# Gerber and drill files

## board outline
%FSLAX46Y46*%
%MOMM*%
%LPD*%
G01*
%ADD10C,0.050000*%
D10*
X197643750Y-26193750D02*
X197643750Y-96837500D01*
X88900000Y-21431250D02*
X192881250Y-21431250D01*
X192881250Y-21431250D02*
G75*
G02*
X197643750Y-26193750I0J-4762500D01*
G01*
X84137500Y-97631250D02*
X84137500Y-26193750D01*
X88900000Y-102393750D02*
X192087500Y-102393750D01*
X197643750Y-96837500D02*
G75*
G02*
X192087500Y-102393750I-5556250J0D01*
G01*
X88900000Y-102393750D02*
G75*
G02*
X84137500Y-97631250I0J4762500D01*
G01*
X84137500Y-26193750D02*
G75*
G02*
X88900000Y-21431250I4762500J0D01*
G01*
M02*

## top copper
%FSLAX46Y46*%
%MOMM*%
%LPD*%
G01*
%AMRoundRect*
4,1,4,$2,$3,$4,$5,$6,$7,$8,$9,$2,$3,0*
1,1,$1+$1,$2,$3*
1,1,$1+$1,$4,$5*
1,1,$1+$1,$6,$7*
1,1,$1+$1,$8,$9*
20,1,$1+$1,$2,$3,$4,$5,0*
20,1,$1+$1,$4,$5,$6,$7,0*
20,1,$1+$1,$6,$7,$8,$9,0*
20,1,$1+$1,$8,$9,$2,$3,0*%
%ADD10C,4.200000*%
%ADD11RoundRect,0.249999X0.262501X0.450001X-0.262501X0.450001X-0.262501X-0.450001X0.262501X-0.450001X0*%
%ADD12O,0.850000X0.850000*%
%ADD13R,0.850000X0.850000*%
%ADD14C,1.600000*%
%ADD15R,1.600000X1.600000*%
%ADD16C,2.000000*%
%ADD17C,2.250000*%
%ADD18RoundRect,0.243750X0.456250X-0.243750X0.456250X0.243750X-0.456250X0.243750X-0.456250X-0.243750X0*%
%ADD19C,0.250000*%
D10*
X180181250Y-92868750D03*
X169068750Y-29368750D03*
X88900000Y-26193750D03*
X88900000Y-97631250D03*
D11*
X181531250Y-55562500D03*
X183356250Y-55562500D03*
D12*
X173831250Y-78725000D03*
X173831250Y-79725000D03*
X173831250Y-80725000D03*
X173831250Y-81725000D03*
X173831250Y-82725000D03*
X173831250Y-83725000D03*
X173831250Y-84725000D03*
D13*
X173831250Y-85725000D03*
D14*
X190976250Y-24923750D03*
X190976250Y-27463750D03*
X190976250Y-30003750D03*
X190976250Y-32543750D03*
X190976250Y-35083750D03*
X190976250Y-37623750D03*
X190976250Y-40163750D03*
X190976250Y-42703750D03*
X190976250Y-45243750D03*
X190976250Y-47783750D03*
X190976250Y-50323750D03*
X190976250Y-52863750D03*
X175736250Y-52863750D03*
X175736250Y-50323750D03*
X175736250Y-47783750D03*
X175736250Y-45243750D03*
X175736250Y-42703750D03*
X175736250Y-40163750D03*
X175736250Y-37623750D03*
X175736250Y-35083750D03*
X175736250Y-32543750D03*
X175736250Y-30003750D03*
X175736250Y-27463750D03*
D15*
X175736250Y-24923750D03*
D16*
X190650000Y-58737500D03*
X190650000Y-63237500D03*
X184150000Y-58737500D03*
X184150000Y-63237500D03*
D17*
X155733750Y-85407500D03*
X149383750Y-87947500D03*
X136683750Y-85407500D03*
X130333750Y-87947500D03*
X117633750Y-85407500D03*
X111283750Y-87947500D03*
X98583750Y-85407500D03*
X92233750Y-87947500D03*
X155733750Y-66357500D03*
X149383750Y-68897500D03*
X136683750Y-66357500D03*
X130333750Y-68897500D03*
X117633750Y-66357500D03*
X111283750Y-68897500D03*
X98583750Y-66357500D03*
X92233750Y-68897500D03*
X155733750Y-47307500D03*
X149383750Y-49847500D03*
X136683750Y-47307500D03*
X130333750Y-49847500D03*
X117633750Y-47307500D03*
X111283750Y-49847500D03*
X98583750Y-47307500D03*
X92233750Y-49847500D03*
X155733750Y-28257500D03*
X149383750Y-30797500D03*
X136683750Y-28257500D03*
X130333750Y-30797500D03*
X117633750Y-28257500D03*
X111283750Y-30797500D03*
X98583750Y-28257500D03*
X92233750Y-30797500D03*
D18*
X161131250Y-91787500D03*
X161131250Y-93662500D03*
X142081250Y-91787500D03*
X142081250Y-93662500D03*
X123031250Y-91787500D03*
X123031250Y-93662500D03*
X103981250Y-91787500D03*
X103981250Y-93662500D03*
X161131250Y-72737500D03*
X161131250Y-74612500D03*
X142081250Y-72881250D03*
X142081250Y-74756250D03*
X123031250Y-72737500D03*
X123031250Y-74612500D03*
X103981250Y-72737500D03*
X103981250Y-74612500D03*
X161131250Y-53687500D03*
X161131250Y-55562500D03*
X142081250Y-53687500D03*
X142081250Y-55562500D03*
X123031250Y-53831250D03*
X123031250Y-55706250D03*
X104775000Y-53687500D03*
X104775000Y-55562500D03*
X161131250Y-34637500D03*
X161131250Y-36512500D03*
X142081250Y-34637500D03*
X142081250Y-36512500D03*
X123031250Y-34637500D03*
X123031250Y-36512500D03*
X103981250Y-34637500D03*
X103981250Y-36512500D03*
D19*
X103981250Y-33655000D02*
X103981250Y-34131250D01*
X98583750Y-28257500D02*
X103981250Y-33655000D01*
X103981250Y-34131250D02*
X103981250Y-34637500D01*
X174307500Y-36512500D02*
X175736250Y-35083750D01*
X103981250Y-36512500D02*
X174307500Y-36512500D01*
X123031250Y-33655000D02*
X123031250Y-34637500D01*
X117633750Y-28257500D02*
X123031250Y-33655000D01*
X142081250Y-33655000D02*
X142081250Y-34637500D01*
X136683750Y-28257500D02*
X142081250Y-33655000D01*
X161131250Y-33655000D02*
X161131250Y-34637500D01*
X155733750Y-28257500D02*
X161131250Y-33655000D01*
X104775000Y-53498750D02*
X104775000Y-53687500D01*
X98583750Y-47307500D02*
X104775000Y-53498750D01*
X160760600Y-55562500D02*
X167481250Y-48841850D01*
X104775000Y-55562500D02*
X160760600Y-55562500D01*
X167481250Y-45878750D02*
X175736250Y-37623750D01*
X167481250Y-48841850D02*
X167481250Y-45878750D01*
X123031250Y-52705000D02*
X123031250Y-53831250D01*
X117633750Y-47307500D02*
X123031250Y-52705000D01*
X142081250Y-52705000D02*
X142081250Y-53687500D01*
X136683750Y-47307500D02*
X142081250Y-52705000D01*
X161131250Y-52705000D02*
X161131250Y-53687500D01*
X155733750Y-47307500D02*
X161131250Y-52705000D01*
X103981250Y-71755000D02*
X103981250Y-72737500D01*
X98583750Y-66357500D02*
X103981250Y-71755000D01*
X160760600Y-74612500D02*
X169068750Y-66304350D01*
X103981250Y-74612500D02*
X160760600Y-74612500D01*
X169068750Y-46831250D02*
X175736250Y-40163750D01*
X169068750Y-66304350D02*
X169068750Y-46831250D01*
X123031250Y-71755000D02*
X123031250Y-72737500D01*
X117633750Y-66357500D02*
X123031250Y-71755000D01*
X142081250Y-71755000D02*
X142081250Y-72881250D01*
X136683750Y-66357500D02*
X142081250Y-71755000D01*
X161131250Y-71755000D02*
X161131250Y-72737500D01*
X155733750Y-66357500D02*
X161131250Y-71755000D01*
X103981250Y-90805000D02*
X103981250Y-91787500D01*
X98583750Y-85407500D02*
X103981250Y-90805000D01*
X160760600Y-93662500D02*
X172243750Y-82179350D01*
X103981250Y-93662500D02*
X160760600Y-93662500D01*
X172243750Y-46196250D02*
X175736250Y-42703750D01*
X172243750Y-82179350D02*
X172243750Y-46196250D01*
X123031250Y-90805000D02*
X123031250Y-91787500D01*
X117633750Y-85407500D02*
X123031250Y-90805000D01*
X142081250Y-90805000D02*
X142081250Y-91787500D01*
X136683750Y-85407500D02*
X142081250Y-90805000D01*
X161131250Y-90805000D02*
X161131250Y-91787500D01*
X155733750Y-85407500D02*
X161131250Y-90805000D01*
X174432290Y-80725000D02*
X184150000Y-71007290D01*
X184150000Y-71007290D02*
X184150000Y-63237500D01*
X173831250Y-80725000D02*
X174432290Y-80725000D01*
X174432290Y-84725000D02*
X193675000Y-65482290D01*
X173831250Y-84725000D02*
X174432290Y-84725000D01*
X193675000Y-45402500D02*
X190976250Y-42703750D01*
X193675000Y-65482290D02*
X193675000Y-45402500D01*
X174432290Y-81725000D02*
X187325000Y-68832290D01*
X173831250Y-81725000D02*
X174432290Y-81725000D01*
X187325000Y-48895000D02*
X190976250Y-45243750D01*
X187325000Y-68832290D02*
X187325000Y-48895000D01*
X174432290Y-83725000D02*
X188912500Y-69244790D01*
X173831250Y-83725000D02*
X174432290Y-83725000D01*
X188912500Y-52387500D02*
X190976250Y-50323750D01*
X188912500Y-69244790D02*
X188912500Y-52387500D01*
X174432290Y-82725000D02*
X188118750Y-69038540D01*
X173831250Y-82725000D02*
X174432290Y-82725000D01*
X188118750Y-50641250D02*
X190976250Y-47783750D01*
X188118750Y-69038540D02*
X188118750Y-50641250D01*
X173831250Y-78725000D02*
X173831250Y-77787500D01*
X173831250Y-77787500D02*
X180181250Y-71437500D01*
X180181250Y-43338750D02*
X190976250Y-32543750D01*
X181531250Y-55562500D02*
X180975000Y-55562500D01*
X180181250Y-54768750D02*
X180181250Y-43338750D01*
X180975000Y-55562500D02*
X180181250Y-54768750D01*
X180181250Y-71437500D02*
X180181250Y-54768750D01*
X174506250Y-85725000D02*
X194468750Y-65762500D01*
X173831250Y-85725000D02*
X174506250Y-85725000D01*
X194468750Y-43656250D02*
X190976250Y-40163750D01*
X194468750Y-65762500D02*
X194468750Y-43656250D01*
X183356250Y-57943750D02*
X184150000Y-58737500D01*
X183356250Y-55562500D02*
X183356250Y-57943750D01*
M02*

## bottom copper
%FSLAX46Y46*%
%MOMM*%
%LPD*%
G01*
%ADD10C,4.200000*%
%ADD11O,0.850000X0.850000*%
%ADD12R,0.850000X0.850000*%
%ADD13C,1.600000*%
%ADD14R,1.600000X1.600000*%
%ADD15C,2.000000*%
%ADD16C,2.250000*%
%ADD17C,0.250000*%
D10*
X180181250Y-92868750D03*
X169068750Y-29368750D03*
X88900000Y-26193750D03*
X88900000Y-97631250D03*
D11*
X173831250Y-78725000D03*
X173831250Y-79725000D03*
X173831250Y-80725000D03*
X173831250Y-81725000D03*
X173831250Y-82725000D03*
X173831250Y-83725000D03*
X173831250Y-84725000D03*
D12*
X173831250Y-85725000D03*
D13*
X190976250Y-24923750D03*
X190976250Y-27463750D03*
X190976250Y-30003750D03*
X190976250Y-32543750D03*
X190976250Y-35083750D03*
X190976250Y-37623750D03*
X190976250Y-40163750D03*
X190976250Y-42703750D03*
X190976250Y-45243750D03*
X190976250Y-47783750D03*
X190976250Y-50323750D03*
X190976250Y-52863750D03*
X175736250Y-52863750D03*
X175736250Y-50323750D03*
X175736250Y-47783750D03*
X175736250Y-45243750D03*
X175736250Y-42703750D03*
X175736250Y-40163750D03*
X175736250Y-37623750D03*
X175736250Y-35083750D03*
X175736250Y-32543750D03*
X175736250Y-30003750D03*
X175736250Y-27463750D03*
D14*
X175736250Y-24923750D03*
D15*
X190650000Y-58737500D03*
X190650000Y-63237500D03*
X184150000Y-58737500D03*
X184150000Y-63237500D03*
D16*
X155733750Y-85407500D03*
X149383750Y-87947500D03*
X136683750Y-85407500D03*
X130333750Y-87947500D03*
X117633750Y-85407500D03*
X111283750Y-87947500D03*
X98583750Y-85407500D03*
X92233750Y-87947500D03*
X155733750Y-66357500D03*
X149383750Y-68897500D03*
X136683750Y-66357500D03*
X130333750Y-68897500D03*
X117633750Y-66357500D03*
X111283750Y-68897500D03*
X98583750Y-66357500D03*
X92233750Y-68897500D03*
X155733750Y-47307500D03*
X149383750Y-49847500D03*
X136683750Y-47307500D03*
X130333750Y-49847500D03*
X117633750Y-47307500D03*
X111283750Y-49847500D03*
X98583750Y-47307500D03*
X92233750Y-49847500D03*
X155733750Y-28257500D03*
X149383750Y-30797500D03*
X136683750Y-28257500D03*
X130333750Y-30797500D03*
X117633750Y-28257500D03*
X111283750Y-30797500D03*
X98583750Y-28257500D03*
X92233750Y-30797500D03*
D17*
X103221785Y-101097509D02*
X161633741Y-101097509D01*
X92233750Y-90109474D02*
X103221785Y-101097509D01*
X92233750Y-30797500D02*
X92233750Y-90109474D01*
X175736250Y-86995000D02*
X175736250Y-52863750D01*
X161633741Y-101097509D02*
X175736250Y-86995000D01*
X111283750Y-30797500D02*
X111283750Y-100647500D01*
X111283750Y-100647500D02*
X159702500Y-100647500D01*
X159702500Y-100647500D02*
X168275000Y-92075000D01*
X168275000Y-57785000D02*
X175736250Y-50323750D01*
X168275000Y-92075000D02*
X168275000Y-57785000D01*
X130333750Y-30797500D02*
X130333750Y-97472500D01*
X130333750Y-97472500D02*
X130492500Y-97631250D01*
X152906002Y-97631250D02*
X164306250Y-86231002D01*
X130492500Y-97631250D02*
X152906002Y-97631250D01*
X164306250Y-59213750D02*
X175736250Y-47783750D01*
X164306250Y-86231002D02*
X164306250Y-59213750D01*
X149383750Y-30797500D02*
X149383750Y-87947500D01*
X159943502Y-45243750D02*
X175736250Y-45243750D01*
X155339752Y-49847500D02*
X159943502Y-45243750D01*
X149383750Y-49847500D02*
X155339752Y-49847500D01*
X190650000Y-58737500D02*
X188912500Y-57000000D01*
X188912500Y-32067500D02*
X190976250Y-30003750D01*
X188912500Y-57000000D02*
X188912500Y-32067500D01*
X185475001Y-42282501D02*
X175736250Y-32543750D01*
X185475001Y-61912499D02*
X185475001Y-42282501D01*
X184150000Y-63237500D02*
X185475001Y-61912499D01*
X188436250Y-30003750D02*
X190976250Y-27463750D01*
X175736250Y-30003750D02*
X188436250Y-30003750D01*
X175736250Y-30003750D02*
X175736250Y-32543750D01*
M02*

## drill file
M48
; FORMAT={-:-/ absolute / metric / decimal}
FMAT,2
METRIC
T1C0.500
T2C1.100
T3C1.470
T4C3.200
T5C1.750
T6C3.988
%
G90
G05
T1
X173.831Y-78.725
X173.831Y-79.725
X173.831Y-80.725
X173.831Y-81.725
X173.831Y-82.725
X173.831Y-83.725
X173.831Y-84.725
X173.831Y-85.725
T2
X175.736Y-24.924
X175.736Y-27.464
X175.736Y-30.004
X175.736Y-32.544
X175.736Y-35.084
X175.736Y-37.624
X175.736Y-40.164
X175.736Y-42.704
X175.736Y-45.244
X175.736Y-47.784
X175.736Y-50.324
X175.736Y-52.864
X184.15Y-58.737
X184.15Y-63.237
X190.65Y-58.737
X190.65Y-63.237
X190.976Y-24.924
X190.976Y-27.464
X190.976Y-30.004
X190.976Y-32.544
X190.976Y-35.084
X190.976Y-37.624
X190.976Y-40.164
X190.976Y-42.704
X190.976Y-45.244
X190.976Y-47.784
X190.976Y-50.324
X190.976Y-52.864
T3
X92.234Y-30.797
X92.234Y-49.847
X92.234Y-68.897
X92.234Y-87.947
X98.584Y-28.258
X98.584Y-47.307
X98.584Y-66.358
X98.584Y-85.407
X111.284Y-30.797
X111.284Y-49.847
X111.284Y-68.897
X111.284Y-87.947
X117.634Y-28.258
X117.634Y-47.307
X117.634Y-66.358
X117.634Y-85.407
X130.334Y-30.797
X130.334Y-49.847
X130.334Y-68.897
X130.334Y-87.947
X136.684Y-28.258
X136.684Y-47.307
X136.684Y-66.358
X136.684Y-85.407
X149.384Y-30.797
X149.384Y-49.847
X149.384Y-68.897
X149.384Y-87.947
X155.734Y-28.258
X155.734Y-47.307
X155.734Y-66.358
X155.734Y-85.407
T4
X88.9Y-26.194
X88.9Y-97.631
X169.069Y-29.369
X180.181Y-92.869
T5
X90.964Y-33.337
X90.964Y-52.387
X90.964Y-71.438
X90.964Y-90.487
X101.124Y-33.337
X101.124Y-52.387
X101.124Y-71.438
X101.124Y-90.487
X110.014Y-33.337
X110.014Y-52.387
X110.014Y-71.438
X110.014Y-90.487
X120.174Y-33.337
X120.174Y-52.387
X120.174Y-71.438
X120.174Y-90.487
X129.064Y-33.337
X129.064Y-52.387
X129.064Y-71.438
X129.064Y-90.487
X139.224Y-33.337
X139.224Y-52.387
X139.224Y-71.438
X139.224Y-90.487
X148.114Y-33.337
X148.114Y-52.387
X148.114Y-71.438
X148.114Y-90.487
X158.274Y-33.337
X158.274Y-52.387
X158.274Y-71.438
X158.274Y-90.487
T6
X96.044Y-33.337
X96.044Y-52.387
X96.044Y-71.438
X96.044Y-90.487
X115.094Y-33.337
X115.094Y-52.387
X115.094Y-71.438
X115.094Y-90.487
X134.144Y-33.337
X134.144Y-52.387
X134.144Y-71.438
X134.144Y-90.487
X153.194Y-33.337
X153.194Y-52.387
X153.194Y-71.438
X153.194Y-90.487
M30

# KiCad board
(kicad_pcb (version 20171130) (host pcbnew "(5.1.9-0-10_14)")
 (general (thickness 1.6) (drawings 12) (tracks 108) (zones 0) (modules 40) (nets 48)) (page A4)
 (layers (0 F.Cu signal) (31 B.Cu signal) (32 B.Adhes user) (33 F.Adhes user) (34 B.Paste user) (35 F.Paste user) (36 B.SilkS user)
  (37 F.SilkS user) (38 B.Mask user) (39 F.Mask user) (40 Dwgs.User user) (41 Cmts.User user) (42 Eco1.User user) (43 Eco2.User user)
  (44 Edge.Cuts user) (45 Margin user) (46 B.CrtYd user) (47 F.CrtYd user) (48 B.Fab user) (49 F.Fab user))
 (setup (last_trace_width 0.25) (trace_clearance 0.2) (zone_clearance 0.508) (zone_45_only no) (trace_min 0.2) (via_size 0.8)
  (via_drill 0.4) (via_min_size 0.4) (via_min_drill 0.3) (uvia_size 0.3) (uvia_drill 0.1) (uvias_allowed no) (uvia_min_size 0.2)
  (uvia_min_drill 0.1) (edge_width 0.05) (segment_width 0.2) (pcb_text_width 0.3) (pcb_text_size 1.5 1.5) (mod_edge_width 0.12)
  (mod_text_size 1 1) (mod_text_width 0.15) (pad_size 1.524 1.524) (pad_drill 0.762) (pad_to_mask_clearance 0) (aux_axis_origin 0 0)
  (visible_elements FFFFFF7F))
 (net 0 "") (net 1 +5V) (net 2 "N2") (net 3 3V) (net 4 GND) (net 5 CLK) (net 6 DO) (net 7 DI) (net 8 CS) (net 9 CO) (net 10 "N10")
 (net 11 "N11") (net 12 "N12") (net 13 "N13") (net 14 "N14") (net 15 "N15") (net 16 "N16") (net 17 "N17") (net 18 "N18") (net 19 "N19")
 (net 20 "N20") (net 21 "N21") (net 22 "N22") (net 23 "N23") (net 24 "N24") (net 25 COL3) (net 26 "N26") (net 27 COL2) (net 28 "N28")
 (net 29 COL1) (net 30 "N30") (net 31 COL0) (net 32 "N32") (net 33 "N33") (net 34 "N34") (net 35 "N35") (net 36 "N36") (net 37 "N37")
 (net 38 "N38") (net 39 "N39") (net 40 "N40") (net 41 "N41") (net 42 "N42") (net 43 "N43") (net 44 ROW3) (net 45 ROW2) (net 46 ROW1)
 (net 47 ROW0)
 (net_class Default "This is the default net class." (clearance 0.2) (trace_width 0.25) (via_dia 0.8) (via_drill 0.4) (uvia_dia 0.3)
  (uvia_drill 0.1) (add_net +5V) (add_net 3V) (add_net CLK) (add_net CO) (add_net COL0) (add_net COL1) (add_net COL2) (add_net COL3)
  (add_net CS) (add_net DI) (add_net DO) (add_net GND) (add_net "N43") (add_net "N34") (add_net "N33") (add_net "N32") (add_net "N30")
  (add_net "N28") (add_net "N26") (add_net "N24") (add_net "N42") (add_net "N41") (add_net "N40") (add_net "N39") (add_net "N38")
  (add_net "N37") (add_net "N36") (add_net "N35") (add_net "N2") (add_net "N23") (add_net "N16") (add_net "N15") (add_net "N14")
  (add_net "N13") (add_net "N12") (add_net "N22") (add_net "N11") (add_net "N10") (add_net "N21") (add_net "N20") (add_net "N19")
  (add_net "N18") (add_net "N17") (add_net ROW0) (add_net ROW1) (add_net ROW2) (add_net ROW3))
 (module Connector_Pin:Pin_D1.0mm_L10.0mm (layer F.Cu) (at 180.18125 92.86875)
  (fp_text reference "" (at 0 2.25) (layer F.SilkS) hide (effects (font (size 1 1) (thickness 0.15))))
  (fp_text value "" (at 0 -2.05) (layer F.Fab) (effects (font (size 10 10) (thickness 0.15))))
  (pad "" thru_hole circle (at 0 0) (size 4.2 4.2) (drill 3.2) (layers *.Cu *.Mask)))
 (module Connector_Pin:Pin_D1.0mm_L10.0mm (layer F.Cu) (at 169.06875 29.36875)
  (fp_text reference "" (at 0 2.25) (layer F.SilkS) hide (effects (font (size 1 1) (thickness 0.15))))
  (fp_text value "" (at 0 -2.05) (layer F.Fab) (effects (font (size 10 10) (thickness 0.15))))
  (pad "" thru_hole circle (at 0 0) (size 4.2 4.2) (drill 3.2) (layers *.Cu *.Mask)))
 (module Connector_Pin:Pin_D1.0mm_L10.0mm (layer F.Cu) (at 88.9 26.19375)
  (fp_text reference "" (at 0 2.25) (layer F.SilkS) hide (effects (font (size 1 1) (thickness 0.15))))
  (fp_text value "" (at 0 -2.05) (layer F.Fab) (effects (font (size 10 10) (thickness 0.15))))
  (pad "" thru_hole circle (at 0 0) (size 4.2 4.2) (drill 3.2) (layers *.Cu *.Mask)))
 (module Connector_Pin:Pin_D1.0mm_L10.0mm (layer F.Cu) (at 88.9 97.63125)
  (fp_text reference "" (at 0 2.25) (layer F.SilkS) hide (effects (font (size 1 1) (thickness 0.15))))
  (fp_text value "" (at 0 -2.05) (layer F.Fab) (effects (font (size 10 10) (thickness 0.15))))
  (pad "" thru_hole circle (at 0 0) (size 4.2 4.2) (drill 3.2) (layers *.Cu *.Mask)))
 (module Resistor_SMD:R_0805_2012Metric (layer F.Cu) (at 182.44375 55.5625 180)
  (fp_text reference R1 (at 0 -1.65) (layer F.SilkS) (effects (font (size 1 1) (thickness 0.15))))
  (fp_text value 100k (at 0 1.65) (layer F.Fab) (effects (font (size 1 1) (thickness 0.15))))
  (pad 2 smd roundrect (at 0.9125 0 180) (size 1.025 1.4) (layers F.Cu F.Paste F.Mask) (roundrect_rratio 0.2439014634146341) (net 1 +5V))
  (pad 1 smd roundrect (at -0.9125 0 180) (size 1.025 1.4) (layers F.Cu F.Paste F.Mask) (roundrect_rratio 0.2439014634146341) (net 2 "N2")))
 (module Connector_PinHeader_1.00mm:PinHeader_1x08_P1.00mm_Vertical (layer F.Cu) (at 173.83125 85.725 180)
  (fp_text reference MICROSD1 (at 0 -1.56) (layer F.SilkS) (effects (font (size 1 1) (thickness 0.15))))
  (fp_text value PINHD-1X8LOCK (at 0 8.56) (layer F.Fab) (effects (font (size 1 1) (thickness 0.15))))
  (pad 8 thru_hole oval (at 0 7 180) (size 0.85 0.85) (drill 0.5) (layers *.Cu *.Mask) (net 1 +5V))
  (pad 7 thru_hole oval (at 0 6 180) (size 0.85 0.85) (drill 0.5) (layers *.Cu *.Mask) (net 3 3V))
  (pad 6 thru_hole oval (at 0 5 180) (size 0.85 0.85) (drill 0.5) (layers *.Cu *.Mask) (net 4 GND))
  (pad 5 thru_hole oval (at 0 4 180) (size 0.85 0.85) (drill 0.5) (layers *.Cu *.Mask) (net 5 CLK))
  (pad 4 thru_hole oval (at 0 3 180) (size 0.85 0.85) (drill 0.5) (layers *.Cu *.Mask) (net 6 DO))
  (pad 3 thru_hole oval (at 0 2 180) (size 0.85 0.85) (drill 0.5) (layers *.Cu *.Mask) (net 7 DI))
  (pad 2 thru_hole oval (at 0 1 180) (size 0.85 0.85) (drill 0.5) (layers *.Cu *.Mask) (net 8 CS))
  (pad 1 thru_hole rect (at 0 0 180) (size 0.85 0.85) (drill 0.5) (layers *.Cu *.Mask) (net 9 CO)))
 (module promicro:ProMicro (layer F.Cu) (at 183.35625 38.89375 270)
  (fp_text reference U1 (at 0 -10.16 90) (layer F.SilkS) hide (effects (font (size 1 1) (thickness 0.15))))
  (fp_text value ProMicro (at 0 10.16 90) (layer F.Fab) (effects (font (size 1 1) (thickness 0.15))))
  (pad 24 thru_hole circle (at -13.97 -7.62 270) (size 1.6 1.6) (drill 1.1) (layers *.Cu *.Mask F.SilkS) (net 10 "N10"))
  (pad 23 thru_hole circle (at -11.43 -7.62 270) (size 1.6 1.6) (drill 1.1) (layers *.Cu *.Mask F.SilkS) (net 4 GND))
  (pad 22 thru_hole circle (at -8.89 -7.62 270) (size 1.6 1.6) (drill 1.1) (layers *.Cu *.Mask F.SilkS) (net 2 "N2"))
  (pad 21 thru_hole circle (at -6.35 -7.62 270) (size 1.6 1.6) (drill 1.1) (layers *.Cu *.Mask F.SilkS) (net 1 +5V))
  (pad 20 thru_hole circle (at -3.81 -7.62 270) (size 1.6 1.6) (drill 1.1) (layers *.Cu *.Mask F.SilkS) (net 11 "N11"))
  (pad 19 thru_hole circle (at -1.27 -7.62 270) (size 1.6 1.6) (drill 1.1) (layers *.Cu *.Mask F.SilkS) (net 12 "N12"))
  (pad 18 thru_hole circle (at 1.27 -7.62 270) (size 1.6 1.6) (drill 1.1) (layers *.Cu *.Mask F.SilkS) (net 9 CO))
  (pad 17 thru_hole circle (at 3.81 -7.62 270) (size 1.6 1.6) (drill 1.1) (layers *.Cu *.Mask F.SilkS) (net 8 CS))
  (pad 16 thru_hole circle (at 6.35 -7.62 270) (size 1.6 1.6) (drill 1.1) (layers *.Cu *.Mask F.SilkS) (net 5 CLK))
  (pad 15 thru_hole circle (at 8.89 -7.62 270) (size 1.6 1.6) (drill 1.1) (layers *.Cu *.Mask F.SilkS) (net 6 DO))
  (pad 14 thru_hole circle (at 11.43 -7.62 270) (size 1.6 1.6) (drill 1.1) (layers *.Cu *.Mask F.SilkS) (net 7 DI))
  (pad 13 thru_hole circle (at 13.97 -7.62 270) (size 1.6 1.6) (drill 1.1) (layers *.Cu *.Mask F.SilkS) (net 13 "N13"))
  (pad 12 thru_hole circle (at 13.97 7.62 270) (size 1.6 1.6) (drill 1.1) (layers *.Cu *.Mask F.SilkS) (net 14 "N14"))
  (pad 11 thru_hole circle (at 11.43 7.62 270) (size 1.6 1.6) (drill 1.1) (layers *.Cu *.Mask F.SilkS) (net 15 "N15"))
  (pad 10 thru_hole circle (at 8.89 7.62 270) (size 1.6 1.6) (drill 1.1) (layers *.Cu *.Mask F.SilkS) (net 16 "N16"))
  (pad 9 thru_hole circle (at 6.35 7.62 270) (size 1.6 1.6) (drill 1.1) (layers *.Cu *.Mask F.SilkS) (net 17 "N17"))
  (pad 8 thru_hole circle (at 3.81 7.62 270) (size 1.6 1.6) (drill 1.1) (layers *.Cu *.Mask F.SilkS) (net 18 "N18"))
  (pad 7 thru_hole circle (at 1.27 7.62 270) (size 1.6 1.6) (drill 1.1) (layers *.Cu *.Mask F.SilkS) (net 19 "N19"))
  (pad 6 thru_hole circle (at -1.27 7.62 270) (size 1.6 1.6) (drill 1.1) (layers *.Cu *.Mask F.SilkS) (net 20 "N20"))
  (pad 5 thru_hole circle (at -3.81 7.62 270) (size 1.6 1.6) (drill 1.1) (layers *.Cu *.Mask F.SilkS) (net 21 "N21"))
  (pad 4 thru_hole circle (at -6.35 7.62 270) (size 1.6 1.6) (drill 1.1) (layers *.Cu *.Mask F.SilkS) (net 4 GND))
  (pad 3 thru_hole circle (at -8.89 7.62 270) (size 1.6 1.6) (drill 1.1) (layers *.Cu *.Mask F.SilkS) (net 4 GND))
  (pad 2 thru_hole circle (at -11.43 7.62 270) (size 1.6 1.6) (drill 1.1) (layers *.Cu *.Mask F.SilkS) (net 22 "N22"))
  (pad 1 thru_hole rect (at -13.97 7.62 270) (size 1.6 1.6) (drill 1.1) (layers *.Cu *.Mask F.SilkS) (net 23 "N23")))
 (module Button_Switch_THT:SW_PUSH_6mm (layer F.Cu) (at 184.15 58.7375)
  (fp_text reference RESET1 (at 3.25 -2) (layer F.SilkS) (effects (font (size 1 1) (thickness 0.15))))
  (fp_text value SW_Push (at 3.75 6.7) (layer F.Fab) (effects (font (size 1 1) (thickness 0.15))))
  (pad 1 thru_hole circle (at 6.5 0 90) (size 2 2) (drill 1.1) (layers *.Cu *.Mask) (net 2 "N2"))
  (pad 2 thru_hole circle (at 6.5 4.5 90) (size 2 2) (drill 1.1) (layers *.Cu *.Mask) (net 4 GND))
  (pad 1 thru_hole circle (at 0 0 90) (size 2 2) (drill 1.1) (layers *.Cu *.Mask) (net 2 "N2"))
  (pad 2 thru_hole circle (at 0 4.5 90) (size 2 2) (drill 1.1) (layers *.Cu *.Mask) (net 4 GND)))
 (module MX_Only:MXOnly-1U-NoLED (layer F.Cu) (at 153.19375 90.4875)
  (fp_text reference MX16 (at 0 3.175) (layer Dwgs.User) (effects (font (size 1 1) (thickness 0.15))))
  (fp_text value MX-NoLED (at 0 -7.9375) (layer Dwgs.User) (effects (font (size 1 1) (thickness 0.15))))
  (pad 2 thru_hole circle (at 2.54 -5.08) (size 2.25 2.25) (drill 1.47) (layers *.Cu B.Mask) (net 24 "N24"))
  (pad "" np_thru_hole circle (at 0 0) (size 3.9878 3.9878) (drill 3.9878) (layers *.Cu *.Mask))
  (pad 1 thru_hole circle (at -3.81 -2.54) (size 2.25 2.25) (drill 1.47) (layers *.Cu B.Mask) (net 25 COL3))
  (pad "" np_thru_hole circle (at -5.08 0 48.0996) (size 1.75 1.75) (drill 1.75) (layers *.Cu *.Mask))
  (pad "" np_thru_hole circle (at 5.08 0 48.0996) (size 1.75 1.75) (drill 1.75) (layers *.Cu *.Mask)))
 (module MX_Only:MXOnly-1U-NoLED (layer F.Cu) (at 134.14375 90.4875)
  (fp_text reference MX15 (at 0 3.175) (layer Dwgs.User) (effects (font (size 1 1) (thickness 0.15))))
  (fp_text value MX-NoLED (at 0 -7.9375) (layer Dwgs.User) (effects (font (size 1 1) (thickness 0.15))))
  (pad 2 thru_hole circle (at 2.54 -5.08) (size 2.25 2.25) (drill 1.47) (layers *.Cu B.Mask) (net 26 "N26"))
  (pad "" np_thru_hole circle (at 0 0) (size 3.9878 3.9878) (drill 3.9878) (layers *.Cu *.Mask))
  (pad 1 thru_hole circle (at -3.81 -2.54) (size 2.25 2.25) (drill 1.47) (layers *.Cu B.Mask) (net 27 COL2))
  (pad "" np_thru_hole circle (at -5.08 0 48.0996) (size 1.75 1.75) (drill 1.75) (layers *.Cu *.Mask))
  (pad "" np_thru_hole circle (at 5.08 0 48.0996) (size 1.75 1.75) (drill 1.75) (layers *.Cu *.Mask)))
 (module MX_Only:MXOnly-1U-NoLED (layer F.Cu) (at 115.09375 90.4875)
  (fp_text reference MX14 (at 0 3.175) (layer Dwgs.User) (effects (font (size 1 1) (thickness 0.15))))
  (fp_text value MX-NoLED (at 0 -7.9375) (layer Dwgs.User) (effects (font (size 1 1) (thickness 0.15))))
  (pad 2 thru_hole circle (at 2.54 -5.08) (size 2.25 2.25) (drill 1.47) (layers *.Cu B.Mask) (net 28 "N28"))
  (pad "" np_thru_hole circle (at 0 0) (size 3.9878 3.9878) (drill 3.9878) (layers *.Cu *.Mask))
  (pad 1 thru_hole circle (at -3.81 -2.54) (size 2.25 2.25) (drill 1.47) (layers *.Cu B.Mask) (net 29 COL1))
  (pad "" np_thru_hole circle (at -5.08 0 48.0996) (size 1.75 1.75) (drill 1.75) (layers *.Cu *.Mask))
  (pad "" np_thru_hole circle (at 5.08 0 48.0996) (size 1.75 1.75) (drill 1.75) (layers *.Cu *.Mask)))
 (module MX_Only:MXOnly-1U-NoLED (layer F.Cu) (at 96.04375 90.4875)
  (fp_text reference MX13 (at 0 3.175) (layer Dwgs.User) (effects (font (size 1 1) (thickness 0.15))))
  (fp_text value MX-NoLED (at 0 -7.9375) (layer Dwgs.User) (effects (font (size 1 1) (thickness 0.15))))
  (pad 2 thru_hole circle (at 2.54 -5.08) (size 2.25 2.25) (drill 1.47) (layers *.Cu B.Mask) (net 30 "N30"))
  (pad "" np_thru_hole circle (at 0 0) (size 3.9878 3.9878) (drill 3.9878) (layers *.Cu *.Mask))
  (pad 1 thru_hole circle (at -3.81 -2.54) (size 2.25 2.25) (drill 1.47) (layers *.Cu B.Mask) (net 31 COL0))
  (pad "" np_thru_hole circle (at -5.08 0 48.0996) (size 1.75 1.75) (drill 1.75) (layers *.Cu *.Mask))
  (pad "" np_thru_hole circle (at 5.08 0 48.0996) (size 1.75 1.75) (drill 1.75) (layers *.Cu *.Mask)))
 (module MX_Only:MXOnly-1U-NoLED (layer F.Cu) (at 153.19375 71.4375)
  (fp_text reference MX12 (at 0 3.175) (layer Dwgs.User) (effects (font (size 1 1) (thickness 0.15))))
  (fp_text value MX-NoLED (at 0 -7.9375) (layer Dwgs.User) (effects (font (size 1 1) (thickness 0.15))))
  (pad 2 thru_hole circle (at 2.54 -5.08) (size 2.25 2.25) (drill 1.47) (layers *.Cu B.Mask) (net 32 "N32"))
  (pad "" np_thru_hole circle (at 0 0) (size 3.9878 3.9878) (drill 3.9878) (layers *.Cu *.Mask))
  (pad 1 thru_hole circle (at -3.81 -2.54) (size 2.25 2.25) (drill 1.47) (layers *.Cu B.Mask) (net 25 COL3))
  (pad "" np_thru_hole circle (at -5.08 0 48.0996) (size 1.75 1.75) (drill 1.75) (layers *.Cu *.Mask))
  (pad "" np_thru_hole circle (at 5.08 0 48.0996) (size 1.75 1.75) (drill 1.75) (layers *.Cu *.Mask)))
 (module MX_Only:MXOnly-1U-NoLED (layer F.Cu) (at 134.14375 71.4375)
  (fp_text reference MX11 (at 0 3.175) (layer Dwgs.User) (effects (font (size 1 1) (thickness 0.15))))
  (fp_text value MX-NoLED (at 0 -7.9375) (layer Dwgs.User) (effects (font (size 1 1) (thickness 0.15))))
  (pad 2 thru_hole circle (at 2.54 -5.08) (size 2.25 2.25) (drill 1.47) (layers *.Cu B.Mask) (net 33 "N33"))
  (pad "" np_thru_hole circle (at 0 0) (size 3.9878 3.9878) (drill 3.9878) (layers *.Cu *.Mask))
  (pad 1 thru_hole circle (at -3.81 -2.54) (size 2.25 2.25) (drill 1.47) (layers *.Cu B.Mask) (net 27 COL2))
  (pad "" np_thru_hole circle (at -5.08 0 48.0996) (size 1.75 1.75) (drill 1.75) (layers *.Cu *.Mask))
  (pad "" np_thru_hole circle (at 5.08 0 48.0996) (size 1.75 1.75) (drill 1.75) (layers *.Cu *.Mask)))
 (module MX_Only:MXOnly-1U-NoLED (layer F.Cu) (at 115.09375 71.4375)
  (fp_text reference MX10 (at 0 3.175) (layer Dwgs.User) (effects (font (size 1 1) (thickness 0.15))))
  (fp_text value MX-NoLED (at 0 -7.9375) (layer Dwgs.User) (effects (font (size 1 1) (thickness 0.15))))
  (pad 2 thru_hole circle (at 2.54 -5.08) (size 2.25 2.25) (drill 1.47) (layers *.Cu B.Mask) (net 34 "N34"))
  (pad "" np_thru_hole circle (at 0 0) (size 3.9878 3.9878) (drill 3.9878) (layers *.Cu *.Mask))
  (pad 1 thru_hole circle (at -3.81 -2.54) (size 2.25 2.25) (drill 1.47) (layers *.Cu B.Mask) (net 29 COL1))
  (pad "" np_thru_hole circle (at -5.08 0 48.0996) (size 1.75 1.75) (drill 1.75) (layers *.Cu *.Mask))
  (pad "" np_thru_hole circle (at 5.08 0 48.0996) (size 1.75 1.75) (drill 1.75) (layers *.Cu *.Mask)))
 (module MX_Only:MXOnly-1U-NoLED (layer F.Cu) (at 96.04375 71.4375)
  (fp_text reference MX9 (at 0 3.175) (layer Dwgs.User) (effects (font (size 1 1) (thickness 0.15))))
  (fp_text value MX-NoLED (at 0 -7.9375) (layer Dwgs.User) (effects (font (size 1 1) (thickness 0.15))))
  (pad 2 thru_hole circle (at 2.54 -5.08) (size 2.25 2.25) (drill 1.47) (layers *.Cu B.Mask) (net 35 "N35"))
  (pad "" np_thru_hole circle (at 0 0) (size 3.9878 3.9878) (drill 3.9878) (layers *.Cu *.Mask))
  (pad 1 thru_hole circle (at -3.81 -2.54) (size 2.25 2.25) (drill 1.47) (layers *.Cu B.Mask) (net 31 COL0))
  (pad "" np_thru_hole circle (at -5.08 0 48.0996) (size 1.75 1.75) (drill 1.75) (layers *.Cu *.Mask))
  (pad "" np_thru_hole circle (at 5.08 0 48.0996) (size 1.75 1.75) (drill 1.75) (layers *.Cu *.Mask)))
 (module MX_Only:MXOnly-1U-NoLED (layer F.Cu) (at 153.19375 52.3875)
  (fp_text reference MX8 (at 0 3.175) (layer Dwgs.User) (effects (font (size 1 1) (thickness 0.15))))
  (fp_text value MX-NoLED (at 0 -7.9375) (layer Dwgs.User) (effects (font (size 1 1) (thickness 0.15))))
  (pad 2 thru_hole circle (at 2.54 -5.08) (size 2.25 2.25) (drill 1.47) (layers *.Cu B.Mask) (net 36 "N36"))
  (pad "" np_thru_hole circle (at 0 0) (size 3.9878 3.9878) (drill 3.9878) (layers *.Cu *.Mask))
  (pad 1 thru_hole circle (at -3.81 -2.54) (size 2.25 2.25) (drill 1.47) (layers *.Cu B.Mask) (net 25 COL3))
  (pad "" np_thru_hole circle (at -5.08 0 48.0996) (size 1.75 1.75) (drill 1.75) (layers *.Cu *.Mask))
  (pad "" np_thru_hole circle (at 5.08 0 48.0996) (size 1.75 1.75) (drill 1.75) (layers *.Cu *.Mask)))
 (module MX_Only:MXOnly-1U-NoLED (layer F.Cu) (at 134.14375 52.3875)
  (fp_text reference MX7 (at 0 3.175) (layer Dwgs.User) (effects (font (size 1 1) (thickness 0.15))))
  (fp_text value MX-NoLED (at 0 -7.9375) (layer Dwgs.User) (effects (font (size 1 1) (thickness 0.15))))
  (pad 2 thru_hole circle (at 2.54 -5.08) (size 2.25 2.25) (drill 1.47) (layers *.Cu B.Mask) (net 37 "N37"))
  (pad "" np_thru_hole circle (at 0 0) (size 3.9878 3.9878) (drill 3.9878) (layers *.Cu *.Mask))
  (pad 1 thru_hole circle (at -3.81 -2.54) (size 2.25 2.25) (drill 1.47) (layers *.Cu B.Mask) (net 27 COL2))
  (pad "" np_thru_hole circle (at -5.08 0 48.0996) (size 1.75 1.75) (drill 1.75) (layers *.Cu *.Mask))
  (pad "" np_thru_hole circle (at 5.08 0 48.0996) (size 1.75 1.75) (drill 1.75) (layers *.Cu *.Mask)))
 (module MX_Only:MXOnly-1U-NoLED (layer F.Cu) (at 115.09375 52.3875)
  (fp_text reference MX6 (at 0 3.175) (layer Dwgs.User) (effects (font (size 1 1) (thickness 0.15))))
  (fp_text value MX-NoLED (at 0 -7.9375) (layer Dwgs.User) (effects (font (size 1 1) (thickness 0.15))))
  (pad 2 thru_hole circle (at 2.54 -5.08) (size 2.25 2.25) (drill 1.47) (layers *.Cu B.Mask) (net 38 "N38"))
  (pad "" np_thru_hole circle (at 0 0) (size 3.9878 3.9878) (drill 3.9878) (layers *.Cu *.Mask))
  (pad 1 thru_hole circle (at -3.81 -2.54) (size 2.25 2.25) (drill 1.47) (layers *.Cu B.Mask) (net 29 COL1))
  (pad "" np_thru_hole circle (at -5.08 0 48.0996) (size 1.75 1.75) (drill 1.75) (layers *.Cu *.Mask))
  (pad "" np_thru_hole circle (at 5.08 0 48.0996) (size 1.75 1.75) (drill 1.75) (layers *.Cu *.Mask)))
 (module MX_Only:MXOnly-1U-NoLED (layer F.Cu) (at 96.04375 52.3875)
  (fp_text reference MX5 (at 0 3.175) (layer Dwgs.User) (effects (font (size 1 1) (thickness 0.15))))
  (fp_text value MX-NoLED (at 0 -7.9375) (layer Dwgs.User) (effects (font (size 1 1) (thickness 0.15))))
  (pad 2 thru_hole circle (at 2.54 -5.08) (size 2.25 2.25) (drill 1.47) (layers *.Cu B.Mask) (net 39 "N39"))
  (pad "" np_thru_hole circle (at 0 0) (size 3.9878 3.9878) (drill 3.9878) (layers *.Cu *.Mask))
  (pad 1 thru_hole circle (at -3.81 -2.54) (size 2.25 2.25) (drill 1.47) (layers *.Cu B.Mask) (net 31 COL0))
  (pad "" np_thru_hole circle (at -5.08 0 48.0996) (size 1.75 1.75) (drill 1.75) (layers *.Cu *.Mask))
  (pad "" np_thru_hole circle (at 5.08 0 48.0996) (size 1.75 1.75) (drill 1.75) (layers *.Cu *.Mask)))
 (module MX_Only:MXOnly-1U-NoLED (layer F.Cu) (at 153.19375 33.3375)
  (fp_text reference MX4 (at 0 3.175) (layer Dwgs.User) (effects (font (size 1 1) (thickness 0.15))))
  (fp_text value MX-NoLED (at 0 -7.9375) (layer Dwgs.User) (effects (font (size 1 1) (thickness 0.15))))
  (pad 2 thru_hole circle (at 2.54 -5.08) (size 2.25 2.25) (drill 1.47) (layers *.Cu B.Mask) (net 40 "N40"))
  (pad "" np_thru_hole circle (at 0 0) (size 3.9878 3.9878) (drill 3.9878) (layers *.Cu *.Mask))
  (pad 1 thru_hole circle (at -3.81 -2.54) (size 2.25 2.25) (drill 1.47) (layers *.Cu B.Mask) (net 25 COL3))
  (pad "" np_thru_hole circle (at -5.08 0 48.0996) (size 1.75 1.75) (drill 1.75) (layers *.Cu *.Mask))
  (pad "" np_thru_hole circle (at 5.08 0 48.0996) (size 1.75 1.75) (drill 1.75) (layers *.Cu *.Mask)))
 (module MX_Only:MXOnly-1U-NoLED (layer F.Cu) (at 134.14375 33.3375)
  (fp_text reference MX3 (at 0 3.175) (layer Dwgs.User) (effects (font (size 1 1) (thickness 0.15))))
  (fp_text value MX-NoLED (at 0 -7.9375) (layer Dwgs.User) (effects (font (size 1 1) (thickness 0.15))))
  (pad 2 thru_hole circle (at 2.54 -5.08) (size 2.25 2.25) (drill 1.47) (layers *.Cu B.Mask) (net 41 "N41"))
  (pad "" np_thru_hole circle (at 0 0) (size 3.9878 3.9878) (drill 3.9878) (layers *.Cu *.Mask))
  (pad 1 thru_hole circle (at -3.81 -2.54) (size 2.25 2.25) (drill 1.47) (layers *.Cu B.Mask) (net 27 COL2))
  (pad "" np_thru_hole circle (at -5.08 0 48.0996) (size 1.75 1.75) (drill 1.75) (layers *.Cu *.Mask))
  (pad "" np_thru_hole circle (at 5.08 0 48.0996) (size 1.75 1.75) (drill 1.75) (layers *.Cu *.Mask)))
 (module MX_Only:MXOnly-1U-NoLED (layer F.Cu) (at 115.09375 33.3375)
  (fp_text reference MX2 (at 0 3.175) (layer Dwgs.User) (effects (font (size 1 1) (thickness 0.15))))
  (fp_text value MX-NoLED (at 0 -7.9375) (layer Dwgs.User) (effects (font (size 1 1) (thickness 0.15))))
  (pad 2 thru_hole circle (at 2.54 -5.08) (size 2.25 2.25) (drill 1.47) (layers *.Cu B.Mask) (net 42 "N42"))
  (pad "" np_thru_hole circle (at 0 0) (size 3.9878 3.9878) (drill 3.9878) (layers *.Cu *.Mask))
  (pad 1 thru_hole circle (at -3.81 -2.54) (size 2.25 2.25) (drill 1.47) (layers *.Cu B.Mask) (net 29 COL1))
  (pad "" np_thru_hole circle (at -5.08 0 48.0996) (size 1.75 1.75) (drill 1.75) (layers *.Cu *.Mask))
  (pad "" np_thru_hole circle (at 5.08 0 48.0996) (size 1.75 1.75) (drill 1.75) (layers *.Cu *.Mask)))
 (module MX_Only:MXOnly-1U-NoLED (layer F.Cu) (at 96.04375 33.3375)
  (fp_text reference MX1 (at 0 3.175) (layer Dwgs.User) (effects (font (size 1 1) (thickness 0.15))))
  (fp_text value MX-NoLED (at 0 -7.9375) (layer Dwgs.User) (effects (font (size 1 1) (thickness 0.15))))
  (pad 2 thru_hole circle (at 2.54 -5.08) (size 2.25 2.25) (drill 1.47) (layers *.Cu B.Mask) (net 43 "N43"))
  (pad "" np_thru_hole circle (at 0 0) (size 3.9878 3.9878) (drill 3.9878) (layers *.Cu *.Mask))
  (pad 1 thru_hole circle (at -3.81 -2.54) (size 2.25 2.25) (drill 1.47) (layers *.Cu B.Mask) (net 31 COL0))
  (pad "" np_thru_hole circle (at -5.08 0 48.0996) (size 1.75 1.75) (drill 1.75) (layers *.Cu *.Mask))
  (pad "" np_thru_hole circle (at 5.08 0 48.0996) (size 1.75 1.75) (drill 1.75) (layers *.Cu *.Mask)))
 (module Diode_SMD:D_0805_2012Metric (layer F.Cu) (at 161.13125 92.725 90)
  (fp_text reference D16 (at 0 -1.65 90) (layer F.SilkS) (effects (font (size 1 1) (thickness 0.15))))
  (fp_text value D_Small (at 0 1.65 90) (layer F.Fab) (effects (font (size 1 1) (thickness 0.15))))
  (pad 2 smd roundrect (at 0.9375 0 90) (size 0.975 1.4) (layers F.Cu F.Paste F.Mask) (roundrect_rratio 0.25) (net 24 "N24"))
  (pad 1 smd roundrect (at -0.9375 0 90) (size 0.975 1.4) (layers F.Cu F.Paste F.Mask) (roundrect_rratio 0.25) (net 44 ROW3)))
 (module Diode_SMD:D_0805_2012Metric (layer F.Cu) (at 142.08125 92.725 90)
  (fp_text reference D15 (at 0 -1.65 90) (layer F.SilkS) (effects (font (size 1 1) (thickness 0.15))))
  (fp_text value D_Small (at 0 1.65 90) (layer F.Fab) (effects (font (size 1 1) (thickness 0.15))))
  (pad 2 smd roundrect (at 0.9375 0 90) (size 0.975 1.4) (layers F.Cu F.Paste F.Mask) (roundrect_rratio 0.25) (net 26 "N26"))
  (pad 1 smd roundrect (at -0.9375 0 90) (size 0.975 1.4) (layers F.Cu F.Paste F.Mask) (roundrect_rratio 0.25) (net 44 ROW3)))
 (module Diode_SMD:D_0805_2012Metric (layer F.Cu) (at 123.03125 92.725 90)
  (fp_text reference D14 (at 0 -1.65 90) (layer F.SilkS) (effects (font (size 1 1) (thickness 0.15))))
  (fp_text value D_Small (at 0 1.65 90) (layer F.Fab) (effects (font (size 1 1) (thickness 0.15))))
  (pad 2 smd roundrect (at 0.9375 0 90) (size 0.975 1.4) (layers F.Cu F.Paste F.Mask) (roundrect_rratio 0.25) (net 28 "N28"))
  (pad 1 smd roundrect (at -0.9375 0 90) (size 0.975 1.4) (layers F.Cu F.Paste F.Mask) (roundrect_rratio 0.25) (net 44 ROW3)))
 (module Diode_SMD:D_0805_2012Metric (layer F.Cu) (at 103.98125 92.725 90)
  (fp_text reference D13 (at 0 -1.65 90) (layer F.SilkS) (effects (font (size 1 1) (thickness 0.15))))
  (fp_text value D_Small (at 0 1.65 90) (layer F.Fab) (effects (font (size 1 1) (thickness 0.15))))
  (pad 2 smd roundrect (at 0.9375 0 90) (size 0.975 1.4) (layers F.Cu F.Paste F.Mask) (roundrect_rratio 0.25) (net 30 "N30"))
  (pad 1 smd roundrect (at -0.9375 0 90) (size 0.975 1.4) (layers F.Cu F.Paste F.Mask) (roundrect_rratio 0.25) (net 44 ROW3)))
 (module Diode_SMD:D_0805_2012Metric (layer F.Cu) (at 161.13125 73.675 90)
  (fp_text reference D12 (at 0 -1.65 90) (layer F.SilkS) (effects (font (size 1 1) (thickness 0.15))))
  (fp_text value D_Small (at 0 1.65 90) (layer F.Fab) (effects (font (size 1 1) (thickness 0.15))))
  (pad 2 smd roundrect (at 0.9375 0 90) (size 0.975 1.4) (layers F.Cu F.Paste F.Mask) (roundrect_rratio 0.25) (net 32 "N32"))
  (pad 1 smd roundrect (at -0.9375 0 90) (size 0.975 1.4) (layers F.Cu F.Paste F.Mask) (roundrect_rratio 0.25) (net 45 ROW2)))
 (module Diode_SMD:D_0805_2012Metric (layer F.Cu) (at 142.08125 73.81875 90)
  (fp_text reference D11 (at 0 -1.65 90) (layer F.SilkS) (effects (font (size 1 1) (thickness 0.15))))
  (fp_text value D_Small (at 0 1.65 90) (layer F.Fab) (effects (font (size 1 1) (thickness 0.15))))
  (pad 2 smd roundrect (at 0.9375 0 90) (size 0.975 1.4) (layers F.Cu F.Paste F.Mask) (roundrect_rratio 0.25) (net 33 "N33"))
  (pad 1 smd roundrect (at -0.9375 0 90) (size 0.975 1.4) (layers F.Cu F.Paste F.Mask) (roundrect_rratio 0.25) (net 45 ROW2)))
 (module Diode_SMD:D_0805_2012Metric (layer F.Cu) (at 123.03125 73.675 90)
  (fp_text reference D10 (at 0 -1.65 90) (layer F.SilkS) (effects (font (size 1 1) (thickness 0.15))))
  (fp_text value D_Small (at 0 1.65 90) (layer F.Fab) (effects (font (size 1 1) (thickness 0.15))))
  (pad 2 smd roundrect (at 0.9375 0 90) (size 0.975 1.4) (layers F.Cu F.Paste F.Mask) (roundrect_rratio 0.25) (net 34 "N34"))
  (pad 1 smd roundrect (at -0.9375 0 90) (size 0.975 1.4) (layers F.Cu F.Paste F.Mask) (roundrect_rratio 0.25) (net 45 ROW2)))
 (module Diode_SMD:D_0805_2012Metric (layer F.Cu) (at 103.98125 73.675 90)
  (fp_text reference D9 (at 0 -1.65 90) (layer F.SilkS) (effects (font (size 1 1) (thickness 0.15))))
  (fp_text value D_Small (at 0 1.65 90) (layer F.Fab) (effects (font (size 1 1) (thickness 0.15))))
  (pad 2 smd roundrect (at 0.9375 0 90) (size 0.975 1.4) (layers F.Cu F.Paste F.Mask) (roundrect_rratio 0.25) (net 35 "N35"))
  (pad 1 smd roundrect (at -0.9375 0 90) (size 0.975 1.4) (layers F.Cu F.Paste F.Mask) (roundrect_rratio 0.25) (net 45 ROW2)))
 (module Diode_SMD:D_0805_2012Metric (layer F.Cu) (at 161.13125 54.625 90)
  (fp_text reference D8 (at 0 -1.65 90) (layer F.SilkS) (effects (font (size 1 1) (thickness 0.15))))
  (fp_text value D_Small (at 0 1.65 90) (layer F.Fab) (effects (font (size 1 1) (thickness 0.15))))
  (pad 2 smd roundrect (at 0.9375 0 90) (size 0.975 1.4) (layers F.Cu F.Paste F.Mask) (roundrect_rratio 0.25) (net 36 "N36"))
  (pad 1 smd roundrect (at -0.9375 0 90) (size 0.975 1.4) (layers F.Cu F.Paste F.Mask) (roundrect_rratio 0.25) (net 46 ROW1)))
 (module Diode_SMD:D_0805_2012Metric (layer F.Cu) (at 142.08125 54.625 90)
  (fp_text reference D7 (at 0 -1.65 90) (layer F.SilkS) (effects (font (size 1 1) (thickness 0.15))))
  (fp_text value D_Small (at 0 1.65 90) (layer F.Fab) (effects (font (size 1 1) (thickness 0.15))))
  (pad 2 smd roundrect (at 0.9375 0 90) (size 0.975 1.4) (layers F.Cu F.Paste F.Mask) (roundrect_rratio 0.25) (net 37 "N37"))
  (pad 1 smd roundrect (at -0.9375 0 90) (size 0.975 1.4) (layers F.Cu F.Paste F.Mask) (roundrect_rratio 0.25) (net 46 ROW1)))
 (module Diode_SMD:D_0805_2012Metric (layer F.Cu) (at 123.03125 54.76875 90)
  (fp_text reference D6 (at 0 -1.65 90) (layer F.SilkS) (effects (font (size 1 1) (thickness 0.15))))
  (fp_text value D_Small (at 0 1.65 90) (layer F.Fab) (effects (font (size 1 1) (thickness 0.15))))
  (pad 2 smd roundrect (at 0.9375 0 90) (size 0.975 1.4) (layers F.Cu F.Paste F.Mask) (roundrect_rratio 0.25) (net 38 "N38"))
  (pad 1 smd roundrect (at -0.9375 0 90) (size 0.975 1.4) (layers F.Cu F.Paste F.Mask) (roundrect_rratio 0.25) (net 46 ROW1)))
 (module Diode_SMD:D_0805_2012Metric (layer F.Cu) (at 104.775 54.625 90)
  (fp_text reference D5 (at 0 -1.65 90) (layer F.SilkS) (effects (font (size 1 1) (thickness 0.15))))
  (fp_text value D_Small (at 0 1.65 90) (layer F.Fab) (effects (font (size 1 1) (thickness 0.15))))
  (pad 2 smd roundrect (at 0.9375 0 90) (size 0.975 1.4) (layers F.Cu F.Paste F.Mask) (roundrect_rratio 0.25) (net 39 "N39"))
  (pad 1 smd roundrect (at -0.9375 0 90) (size 0.975 1.4) (layers F.Cu F.Paste F.Mask) (roundrect_rratio 0.25) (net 46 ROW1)))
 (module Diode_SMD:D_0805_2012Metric (layer F.Cu) (at 161.13125 35.575 90)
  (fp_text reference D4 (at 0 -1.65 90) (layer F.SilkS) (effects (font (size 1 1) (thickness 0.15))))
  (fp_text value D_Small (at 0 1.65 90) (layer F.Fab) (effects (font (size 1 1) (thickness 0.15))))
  (pad 2 smd roundrect (at 0.9375 0 90) (size 0.975 1.4) (layers F.Cu F.Paste F.Mask) (roundrect_rratio 0.25) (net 40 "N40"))
  (pad 1 smd roundrect (at -0.9375 0 90) (size 0.975 1.4) (layers F.Cu F.Paste F.Mask) (roundrect_rratio 0.25) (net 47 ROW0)))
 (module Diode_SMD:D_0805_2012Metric (layer F.Cu) (at 142.08125 35.575 90)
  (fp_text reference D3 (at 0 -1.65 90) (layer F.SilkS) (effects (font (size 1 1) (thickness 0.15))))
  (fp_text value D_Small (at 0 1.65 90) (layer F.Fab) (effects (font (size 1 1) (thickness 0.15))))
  (pad 2 smd roundrect (at 0.9375 0 90) (size 0.975 1.4) (layers F.Cu F.Paste F.Mask) (roundrect_rratio 0.25) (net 41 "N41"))
  (pad 1 smd roundrect (at -0.9375 0 90) (size 0.975 1.4) (layers F.Cu F.Paste F.Mask) (roundrect_rratio 0.25) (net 47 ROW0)))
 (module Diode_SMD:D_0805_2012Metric (layer F.Cu) (at 123.03125 35.575 90)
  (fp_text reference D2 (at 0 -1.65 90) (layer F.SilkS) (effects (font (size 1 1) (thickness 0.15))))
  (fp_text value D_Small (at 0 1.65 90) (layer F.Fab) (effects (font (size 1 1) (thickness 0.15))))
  (pad 2 smd roundrect (at 0.9375 0 90) (size 0.975 1.4) (layers F.Cu F.Paste F.Mask) (roundrect_rratio 0.25) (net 42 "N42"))
  (pad 1 smd roundrect (at -0.9375 0 90) (size 0.975 1.4) (layers F.Cu F.Paste F.Mask) (roundrect_rratio 0.25) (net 47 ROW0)))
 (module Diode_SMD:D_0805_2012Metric (layer F.Cu) (at 103.98125 35.575 90)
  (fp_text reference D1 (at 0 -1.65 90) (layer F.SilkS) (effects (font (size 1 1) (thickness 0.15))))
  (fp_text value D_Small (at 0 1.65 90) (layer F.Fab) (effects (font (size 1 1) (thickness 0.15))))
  (pad 2 smd roundrect (at 0.9375 0 90) (size 0.975 1.4) (layers F.Cu F.Paste F.Mask) (roundrect_rratio 0.25) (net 43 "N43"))
  (pad 1 smd roundrect (at -0.9375 0 90) (size 0.975 1.4) (layers F.Cu F.Paste F.Mask) (roundrect_rratio 0.25) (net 47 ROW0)))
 (gr_line (start 197.64375 26.19375) (end 197.64375 96.8375) (layer Edge.Cuts) (width 0.05))
 (gr_line (start 88.9 21.43125) (end 192.88125 21.43125) (layer Edge.Cuts) (width 0.05))
 (gr_arc (start 192.88125 26.19375) (end 197.64375 26.19375) (angle -90) (layer Edge.Cuts) (width 0.05))
 (gr_line (start 84.1375 97.63125) (end 84.1375 26.19375) (layer Edge.Cuts) (width 0.05))
 (gr_line (start 88.9 102.39375) (end 192.0875 102.39375) (layer Edge.Cuts) (width 0.05))
 (gr_arc (start 192.0875 96.8375) (end 192.0875 102.39375) (angle -90) (layer Edge.Cuts) (width 0.05))
 (gr_arc (start 88.9 97.63125) (end 84.1375 97.63125) (angle -90) (layer Edge.Cuts) (width 0.05))
 (gr_arc (start 88.9 26.19375) (end 88.9 21.43125) (angle -90) (layer Edge.Cuts) (width 0.05))
 (segment (start 103.98125 33.655) (end 103.98125 34.13125) (width 0.25) (layer F.Cu) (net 43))
 (segment (start 98.58375 28.2575) (end 103.98125 33.655) (width 0.25) (layer F.Cu) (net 43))
 (segment (start 103.98125 34.13125) (end 103.98125 34.6375) (width 0.25) (layer F.Cu) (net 43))
 (segment (start 174.3075 36.5125) (end 175.73625 35.08375) (width 0.25) (layer F.Cu) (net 47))
 (segment (start 103.98125 36.5125) (end 174.3075 36.5125) (width 0.25) (layer F.Cu) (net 47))
 (segment (start 123.03125 33.655) (end 123.03125 34.6375) (width 0.25) (layer F.Cu) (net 42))
 (segment (start 117.63375 28.2575) (end 123.03125 33.655) (width 0.25) (layer F.Cu) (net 42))
 (segment (start 142.08125 33.655) (end 142.08125 34.6375) (width 0.25) (layer F.Cu) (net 41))
 (segment (start 136.68375 28.2575) (end 142.08125 33.655) (width 0.25) (layer F.Cu) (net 41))
 (segment (start 161.13125 33.655) (end 161.13125 34.6375) (width 0.25) (layer F.Cu) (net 40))
 (segment (start 155.73375 28.2575) (end 161.13125 33.655) (width 0.25) (layer F.Cu) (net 40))
 (segment (start 104.775 53.49875) (end 104.775 53.6875) (width 0.25) (layer F.Cu) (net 39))
 (segment (start 98.58375 47.3075) (end 104.775 53.49875) (width 0.25) (layer F.Cu) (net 39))
 (segment (start 160.7606 55.5625) (end 167.48125 48.84185) (width 0.25) (layer F.Cu) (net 46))
 (segment (start 104.775 55.5625) (end 160.7606 55.5625) (width 0.25) (layer F.Cu) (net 46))
 (segment (start 167.48125 45.87875) (end 175.73625 37.62375) (width 0.25) (layer F.Cu) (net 46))
 (segment (start 167.48125 48.84185) (end 167.48125 45.87875) (width 0.25) (layer F.Cu) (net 46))
 (segment (start 123.03125 52.705) (end 123.03125 53.83125) (width 0.25) (layer F.Cu) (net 38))
 (segment (start 117.63375 47.3075) (end 123.03125 52.705) (width 0.25) (layer F.Cu) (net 38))
 (segment (start 142.08125 52.705) (end 142.08125 53.6875) (width 0.25) (layer F.Cu) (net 37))
 (segment (start 136.68375 47.3075) (end 142.08125 52.705) (width 0.25) (layer F.Cu) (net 37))
 (segment (start 161.13125 52.705) (end 161.13125 53.6875) (width 0.25) (layer F.Cu) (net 36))
 (segment (start 155.73375 47.3075) (end 161.13125 52.705) (width 0.25) (layer F.Cu) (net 36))
 (segment (start 103.98125 71.755) (end 103.98125 72.7375) (width 0.25) (layer F.Cu) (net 35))
 (segment (start 98.58375 66.3575) (end 103.98125 71.755) (width 0.25) (layer F.Cu) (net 35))
 (segment (start 160.7606 74.6125) (end 169.06875 66.30435) (width 0.25) (layer F.Cu) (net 45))
 (segment (start 103.98125 74.6125) (end 160.7606 74.6125) (width 0.25) (layer F.Cu) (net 45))
 (segment (start 169.06875 46.83125) (end 175.73625 40.16375) (width 0.25) (layer F.Cu) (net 45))
 (segment (start 169.06875 66.30435) (end 169.06875 46.83125) (width 0.25) (layer F.Cu) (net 45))
 (segment (start 123.03125 71.755) (end 123.03125 72.7375) (width 0.25) (layer F.Cu) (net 34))
 (segment (start 117.63375 66.3575) (end 123.03125 71.755) (width 0.25) (layer F.Cu) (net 34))
 (segment (start 142.08125 71.755) (end 142.08125 72.88125) (width 0.25) (layer F.Cu) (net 33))
 (segment (start 136.68375 66.3575) (end 142.08125 71.755) (width 0.25) (layer F.Cu) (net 33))
 (segment (start 161.13125 71.755) (end 161.13125 72.7375) (width 0.25) (layer F.Cu) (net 32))
 (segment (start 155.73375 66.3575) (end 161.13125 71.755) (width 0.25) (layer F.Cu) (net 32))
 (segment (start 103.98125 90.805) (end 103.98125 91.7875) (width 0.25) (layer F.Cu) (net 30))
 (segment (start 98.58375 85.4075) (end 103.98125 90.805) (width 0.25) (layer F.Cu) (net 30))
 (segment (start 160.7606 93.6625) (end 172.24375 82.17935) (width 0.25) (layer F.Cu) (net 44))
 (segment (start 103.98125 93.6625) (end 160.7606 93.6625) (width 0.25) (layer F.Cu) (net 44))
 (segment (start 172.24375 46.19625) (end 175.73625 42.70375) (width 0.25) (layer F.Cu) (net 44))
 (segment (start 172.24375 82.17935) (end 172.24375 46.19625) (width 0.25) (layer F.Cu) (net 44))
 (segment (start 123.03125 90.805) (end 123.03125 91.7875) (width 0.25) (layer F.Cu) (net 28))
 (segment (start 117.63375 85.4075) (end 123.03125 90.805) (width 0.25) (layer F.Cu) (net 28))
 (segment (start 142.08125 90.805) (end 142.08125 91.7875) (width 0.25) (layer F.Cu) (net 26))
 (segment (start 136.68375 85.4075) (end 142.08125 90.805) (width 0.25) (layer F.Cu) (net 26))
 (segment (start 161.13125 90.805) (end 161.13125 91.7875) (width 0.25) (layer F.Cu) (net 24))
 (segment (start 155.73375 85.4075) (end 161.13125 90.805) (width 0.25) (layer F.Cu) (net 24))
 (segment (start 103.221785 101.097509) (end 161.633741 101.097509) (width 0.25) (layer B.Cu) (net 31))
 (segment (start 92.23375 90.109474) (end 103.221785 101.097509) (width 0.25) (layer B.Cu) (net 31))
 (segment (start 92.23375 30.7975) (end 92.23375 90.109474) (width 0.25) (layer B.Cu) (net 31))
 (segment (start 175.73625 86.995) (end 175.73625 52.86375) (width 0.25) (layer B.Cu) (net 31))
 (segment (start 161.633741 101.097509) (end 175.73625 86.995) (width 0.25) (layer B.Cu) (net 31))
 (segment (start 111.28375 30.7975) (end 111.28375 100.6475) (width 0.25) (layer B.Cu) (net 29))
 (segment (start 111.28375 100.6475) (end 159.7025 100.6475) (width 0.25) (layer B.Cu) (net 29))
 (segment (start 159.7025 100.6475) (end 168.275 92.075) (width 0.25) (layer B.Cu) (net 29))
 (segment (start 168.275 57.785) (end 175.73625 50.32375) (width 0.25) (layer B.Cu) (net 29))
 (segment (start 168.275 92.075) (end 168.275 57.785) (width 0.25) (layer B.Cu) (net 29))
 (segment (start 130.33375 30.7975) (end 130.33375 97.4725) (width 0.25) (layer B.Cu) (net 27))
 (segment (start 130.33375 97.4725) (end 130.4925 97.63125) (width 0.25) (layer B.Cu) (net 27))
 (segment (start 152.906002 97.63125) (end 164.30625 86.231002) (width 0.25) (layer B.Cu) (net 27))
 (segment (start 130.4925 97.63125) (end 152.906002 97.63125) (width 0.25) (layer B.Cu) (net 27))
 (segment (start 164.30625 59.21375) (end 175.73625 47.78375) (width 0.25) (layer B.Cu) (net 27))
 (segment (start 164.30625 86.231002) (end 164.30625 59.21375) (width 0.25) (layer B.Cu) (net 27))
 (segment (start 149.38375 30.7975) (end 149.38375 87.9475) (width 0.25) (layer B.Cu) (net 25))
 (segment (start 159.943502 45.24375) (end 175.73625 45.24375) (width 0.25) (layer B.Cu) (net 25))
 (segment (start 155.339752 49.8475) (end 159.943502 45.24375) (width 0.25) (layer B.Cu) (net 25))
 (segment (start 149.38375 49.8475) (end 155.339752 49.8475) (width 0.25) (layer B.Cu) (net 25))
 (segment (start 190.65 58.7375) (end 188.9125 57) (width 0.25) (layer B.Cu) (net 2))
 (segment (start 188.9125 32.0675) (end 190.97625 30.00375) (width 0.25) (layer B.Cu) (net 2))
 (segment (start 188.9125 57) (end 188.9125 32.0675) (width 0.25) (layer B.Cu) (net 2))
 (segment (start 185.475001 42.282501) (end 175.73625 32.54375) (width 0.25) (layer B.Cu) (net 4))
 (segment (start 185.475001 61.912499) (end 185.475001 42.282501) (width 0.25) (layer B.Cu) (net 4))
 (segment (start 184.15 63.2375) (end 185.475001 61.912499) (width 0.25) (layer B.Cu) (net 4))
 (segment (start 188.43625 30.00375) (end 190.97625 27.46375) (width 0.25) (layer B.Cu) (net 4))
 (segment (start 175.73625 30.00375) (end 188.43625 30.00375) (width 0.25) (layer B.Cu) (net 4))
 (segment (start 175.73625 30.00375) (end 175.73625 32.54375) (width 0.25) (layer B.Cu) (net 4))
 (segment (start 174.43229 80.725) (end 184.15 71.00729) (width 0.25) (layer F.Cu) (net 4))
 (segment (start 184.15 71.00729) (end 184.15 63.2375) (width 0.25) (layer F.Cu) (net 4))
 (segment (start 173.83125 80.725) (end 174.43229 80.725) (width 0.25) (layer F.Cu) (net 4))
 (segment (start 174.43229 84.725) (end 193.675 65.48229) (width 0.25) (layer F.Cu) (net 8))
 (segment (start 173.83125 84.725) (end 174.43229 84.725) (width 0.25) (layer F.Cu) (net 8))
 (segment (start 193.675 45.4025) (end 190.97625 42.70375) (width 0.25) (layer F.Cu) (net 8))
 (segment (start 193.675 65.48229) (end 193.675 45.4025) (width 0.25) (layer F.Cu) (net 8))
 (segment (start 174.43229 81.725) (end 187.325 68.83229) (width 0.25) (layer F.Cu) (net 5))
 (segment (start 173.83125 81.725) (end 174.43229 81.725) (width 0.25) (layer F.Cu) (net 5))
 (segment (start 187.325 48.895) (end 190.97625 45.24375) (width 0.25) (layer F.Cu) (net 5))
 (segment (start 187.325 68.83229) (end 187.325 48.895) (width 0.25) (layer F.Cu) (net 5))
 (segment (start 174.43229 83.725) (end 188.9125 69.24479) (width 0.25) (layer F.Cu) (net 7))
 (segment (start 173.83125 83.725) (end 174.43229 83.725) (width 0.25) (layer F.Cu) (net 7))
 (segment (start 188.9125 52.3875) (end 190.97625 50.32375) (width 0.25) (layer F.Cu) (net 7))
 (segment (start 188.9125 69.24479) (end 188.9125 52.3875) (width 0.25) (layer F.Cu) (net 7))
 (segment (start 174.43229 82.725) (end 188.11875 69.03854) (width 0.25) (layer F.Cu) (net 6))
 (segment (start 173.83125 82.725) (end 174.43229 82.725) (width 0.25) (layer F.Cu) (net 6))
 (segment (start 188.11875 50.64125) (end 190.97625 47.78375) (width 0.25) (layer F.Cu) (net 6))
 (segment (start 188.11875 69.03854) (end 188.11875 50.64125) (width 0.25) (layer F.Cu) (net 6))
 (segment (start 173.83125 78.725) (end 173.83125 77.7875) (width 0.25) (layer F.Cu) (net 1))
 (segment (start 173.83125 77.7875) (end 180.18125 71.4375) (width 0.25) (layer F.Cu) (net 1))
 (segment (start 180.18125 43.33875) (end 190.97625 32.54375) (width 0.25) (layer F.Cu) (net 1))
 (segment (start 181.53125 55.5625) (end 180.975 55.5625) (width 0.25) (layer F.Cu) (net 1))
 (segment (start 180.18125 54.76875) (end 180.18125 43.33875) (width 0.25) (layer F.Cu) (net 1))
 (segment (start 180.975 55.5625) (end 180.18125 54.76875) (width 0.25) (layer F.Cu) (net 1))
 (segment (start 180.18125 71.4375) (end 180.18125 54.76875) (width 0.25) (layer F.Cu) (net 1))
 (segment (start 174.50625 85.725) (end 194.46875 65.7625) (width 0.25) (layer F.Cu) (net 9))
 (segment (start 173.83125 85.725) (end 174.50625 85.725) (width 0.25) (layer F.Cu) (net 9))
 (segment (start 194.46875 43.65625) (end 190.97625 40.16375) (width 0.25) (layer F.Cu) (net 9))
 (segment (start 194.46875 65.7625) (end 194.46875 43.65625) (width 0.25) (layer F.Cu) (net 9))
 (segment (start 183.35625 57.94375) (end 184.15 58.7375) (width 0.25) (layer F.Cu) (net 2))
 (segment (start 183.35625 55.5625) (end 183.35625 57.94375) (width 0.25) (layer F.Cu) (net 2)))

